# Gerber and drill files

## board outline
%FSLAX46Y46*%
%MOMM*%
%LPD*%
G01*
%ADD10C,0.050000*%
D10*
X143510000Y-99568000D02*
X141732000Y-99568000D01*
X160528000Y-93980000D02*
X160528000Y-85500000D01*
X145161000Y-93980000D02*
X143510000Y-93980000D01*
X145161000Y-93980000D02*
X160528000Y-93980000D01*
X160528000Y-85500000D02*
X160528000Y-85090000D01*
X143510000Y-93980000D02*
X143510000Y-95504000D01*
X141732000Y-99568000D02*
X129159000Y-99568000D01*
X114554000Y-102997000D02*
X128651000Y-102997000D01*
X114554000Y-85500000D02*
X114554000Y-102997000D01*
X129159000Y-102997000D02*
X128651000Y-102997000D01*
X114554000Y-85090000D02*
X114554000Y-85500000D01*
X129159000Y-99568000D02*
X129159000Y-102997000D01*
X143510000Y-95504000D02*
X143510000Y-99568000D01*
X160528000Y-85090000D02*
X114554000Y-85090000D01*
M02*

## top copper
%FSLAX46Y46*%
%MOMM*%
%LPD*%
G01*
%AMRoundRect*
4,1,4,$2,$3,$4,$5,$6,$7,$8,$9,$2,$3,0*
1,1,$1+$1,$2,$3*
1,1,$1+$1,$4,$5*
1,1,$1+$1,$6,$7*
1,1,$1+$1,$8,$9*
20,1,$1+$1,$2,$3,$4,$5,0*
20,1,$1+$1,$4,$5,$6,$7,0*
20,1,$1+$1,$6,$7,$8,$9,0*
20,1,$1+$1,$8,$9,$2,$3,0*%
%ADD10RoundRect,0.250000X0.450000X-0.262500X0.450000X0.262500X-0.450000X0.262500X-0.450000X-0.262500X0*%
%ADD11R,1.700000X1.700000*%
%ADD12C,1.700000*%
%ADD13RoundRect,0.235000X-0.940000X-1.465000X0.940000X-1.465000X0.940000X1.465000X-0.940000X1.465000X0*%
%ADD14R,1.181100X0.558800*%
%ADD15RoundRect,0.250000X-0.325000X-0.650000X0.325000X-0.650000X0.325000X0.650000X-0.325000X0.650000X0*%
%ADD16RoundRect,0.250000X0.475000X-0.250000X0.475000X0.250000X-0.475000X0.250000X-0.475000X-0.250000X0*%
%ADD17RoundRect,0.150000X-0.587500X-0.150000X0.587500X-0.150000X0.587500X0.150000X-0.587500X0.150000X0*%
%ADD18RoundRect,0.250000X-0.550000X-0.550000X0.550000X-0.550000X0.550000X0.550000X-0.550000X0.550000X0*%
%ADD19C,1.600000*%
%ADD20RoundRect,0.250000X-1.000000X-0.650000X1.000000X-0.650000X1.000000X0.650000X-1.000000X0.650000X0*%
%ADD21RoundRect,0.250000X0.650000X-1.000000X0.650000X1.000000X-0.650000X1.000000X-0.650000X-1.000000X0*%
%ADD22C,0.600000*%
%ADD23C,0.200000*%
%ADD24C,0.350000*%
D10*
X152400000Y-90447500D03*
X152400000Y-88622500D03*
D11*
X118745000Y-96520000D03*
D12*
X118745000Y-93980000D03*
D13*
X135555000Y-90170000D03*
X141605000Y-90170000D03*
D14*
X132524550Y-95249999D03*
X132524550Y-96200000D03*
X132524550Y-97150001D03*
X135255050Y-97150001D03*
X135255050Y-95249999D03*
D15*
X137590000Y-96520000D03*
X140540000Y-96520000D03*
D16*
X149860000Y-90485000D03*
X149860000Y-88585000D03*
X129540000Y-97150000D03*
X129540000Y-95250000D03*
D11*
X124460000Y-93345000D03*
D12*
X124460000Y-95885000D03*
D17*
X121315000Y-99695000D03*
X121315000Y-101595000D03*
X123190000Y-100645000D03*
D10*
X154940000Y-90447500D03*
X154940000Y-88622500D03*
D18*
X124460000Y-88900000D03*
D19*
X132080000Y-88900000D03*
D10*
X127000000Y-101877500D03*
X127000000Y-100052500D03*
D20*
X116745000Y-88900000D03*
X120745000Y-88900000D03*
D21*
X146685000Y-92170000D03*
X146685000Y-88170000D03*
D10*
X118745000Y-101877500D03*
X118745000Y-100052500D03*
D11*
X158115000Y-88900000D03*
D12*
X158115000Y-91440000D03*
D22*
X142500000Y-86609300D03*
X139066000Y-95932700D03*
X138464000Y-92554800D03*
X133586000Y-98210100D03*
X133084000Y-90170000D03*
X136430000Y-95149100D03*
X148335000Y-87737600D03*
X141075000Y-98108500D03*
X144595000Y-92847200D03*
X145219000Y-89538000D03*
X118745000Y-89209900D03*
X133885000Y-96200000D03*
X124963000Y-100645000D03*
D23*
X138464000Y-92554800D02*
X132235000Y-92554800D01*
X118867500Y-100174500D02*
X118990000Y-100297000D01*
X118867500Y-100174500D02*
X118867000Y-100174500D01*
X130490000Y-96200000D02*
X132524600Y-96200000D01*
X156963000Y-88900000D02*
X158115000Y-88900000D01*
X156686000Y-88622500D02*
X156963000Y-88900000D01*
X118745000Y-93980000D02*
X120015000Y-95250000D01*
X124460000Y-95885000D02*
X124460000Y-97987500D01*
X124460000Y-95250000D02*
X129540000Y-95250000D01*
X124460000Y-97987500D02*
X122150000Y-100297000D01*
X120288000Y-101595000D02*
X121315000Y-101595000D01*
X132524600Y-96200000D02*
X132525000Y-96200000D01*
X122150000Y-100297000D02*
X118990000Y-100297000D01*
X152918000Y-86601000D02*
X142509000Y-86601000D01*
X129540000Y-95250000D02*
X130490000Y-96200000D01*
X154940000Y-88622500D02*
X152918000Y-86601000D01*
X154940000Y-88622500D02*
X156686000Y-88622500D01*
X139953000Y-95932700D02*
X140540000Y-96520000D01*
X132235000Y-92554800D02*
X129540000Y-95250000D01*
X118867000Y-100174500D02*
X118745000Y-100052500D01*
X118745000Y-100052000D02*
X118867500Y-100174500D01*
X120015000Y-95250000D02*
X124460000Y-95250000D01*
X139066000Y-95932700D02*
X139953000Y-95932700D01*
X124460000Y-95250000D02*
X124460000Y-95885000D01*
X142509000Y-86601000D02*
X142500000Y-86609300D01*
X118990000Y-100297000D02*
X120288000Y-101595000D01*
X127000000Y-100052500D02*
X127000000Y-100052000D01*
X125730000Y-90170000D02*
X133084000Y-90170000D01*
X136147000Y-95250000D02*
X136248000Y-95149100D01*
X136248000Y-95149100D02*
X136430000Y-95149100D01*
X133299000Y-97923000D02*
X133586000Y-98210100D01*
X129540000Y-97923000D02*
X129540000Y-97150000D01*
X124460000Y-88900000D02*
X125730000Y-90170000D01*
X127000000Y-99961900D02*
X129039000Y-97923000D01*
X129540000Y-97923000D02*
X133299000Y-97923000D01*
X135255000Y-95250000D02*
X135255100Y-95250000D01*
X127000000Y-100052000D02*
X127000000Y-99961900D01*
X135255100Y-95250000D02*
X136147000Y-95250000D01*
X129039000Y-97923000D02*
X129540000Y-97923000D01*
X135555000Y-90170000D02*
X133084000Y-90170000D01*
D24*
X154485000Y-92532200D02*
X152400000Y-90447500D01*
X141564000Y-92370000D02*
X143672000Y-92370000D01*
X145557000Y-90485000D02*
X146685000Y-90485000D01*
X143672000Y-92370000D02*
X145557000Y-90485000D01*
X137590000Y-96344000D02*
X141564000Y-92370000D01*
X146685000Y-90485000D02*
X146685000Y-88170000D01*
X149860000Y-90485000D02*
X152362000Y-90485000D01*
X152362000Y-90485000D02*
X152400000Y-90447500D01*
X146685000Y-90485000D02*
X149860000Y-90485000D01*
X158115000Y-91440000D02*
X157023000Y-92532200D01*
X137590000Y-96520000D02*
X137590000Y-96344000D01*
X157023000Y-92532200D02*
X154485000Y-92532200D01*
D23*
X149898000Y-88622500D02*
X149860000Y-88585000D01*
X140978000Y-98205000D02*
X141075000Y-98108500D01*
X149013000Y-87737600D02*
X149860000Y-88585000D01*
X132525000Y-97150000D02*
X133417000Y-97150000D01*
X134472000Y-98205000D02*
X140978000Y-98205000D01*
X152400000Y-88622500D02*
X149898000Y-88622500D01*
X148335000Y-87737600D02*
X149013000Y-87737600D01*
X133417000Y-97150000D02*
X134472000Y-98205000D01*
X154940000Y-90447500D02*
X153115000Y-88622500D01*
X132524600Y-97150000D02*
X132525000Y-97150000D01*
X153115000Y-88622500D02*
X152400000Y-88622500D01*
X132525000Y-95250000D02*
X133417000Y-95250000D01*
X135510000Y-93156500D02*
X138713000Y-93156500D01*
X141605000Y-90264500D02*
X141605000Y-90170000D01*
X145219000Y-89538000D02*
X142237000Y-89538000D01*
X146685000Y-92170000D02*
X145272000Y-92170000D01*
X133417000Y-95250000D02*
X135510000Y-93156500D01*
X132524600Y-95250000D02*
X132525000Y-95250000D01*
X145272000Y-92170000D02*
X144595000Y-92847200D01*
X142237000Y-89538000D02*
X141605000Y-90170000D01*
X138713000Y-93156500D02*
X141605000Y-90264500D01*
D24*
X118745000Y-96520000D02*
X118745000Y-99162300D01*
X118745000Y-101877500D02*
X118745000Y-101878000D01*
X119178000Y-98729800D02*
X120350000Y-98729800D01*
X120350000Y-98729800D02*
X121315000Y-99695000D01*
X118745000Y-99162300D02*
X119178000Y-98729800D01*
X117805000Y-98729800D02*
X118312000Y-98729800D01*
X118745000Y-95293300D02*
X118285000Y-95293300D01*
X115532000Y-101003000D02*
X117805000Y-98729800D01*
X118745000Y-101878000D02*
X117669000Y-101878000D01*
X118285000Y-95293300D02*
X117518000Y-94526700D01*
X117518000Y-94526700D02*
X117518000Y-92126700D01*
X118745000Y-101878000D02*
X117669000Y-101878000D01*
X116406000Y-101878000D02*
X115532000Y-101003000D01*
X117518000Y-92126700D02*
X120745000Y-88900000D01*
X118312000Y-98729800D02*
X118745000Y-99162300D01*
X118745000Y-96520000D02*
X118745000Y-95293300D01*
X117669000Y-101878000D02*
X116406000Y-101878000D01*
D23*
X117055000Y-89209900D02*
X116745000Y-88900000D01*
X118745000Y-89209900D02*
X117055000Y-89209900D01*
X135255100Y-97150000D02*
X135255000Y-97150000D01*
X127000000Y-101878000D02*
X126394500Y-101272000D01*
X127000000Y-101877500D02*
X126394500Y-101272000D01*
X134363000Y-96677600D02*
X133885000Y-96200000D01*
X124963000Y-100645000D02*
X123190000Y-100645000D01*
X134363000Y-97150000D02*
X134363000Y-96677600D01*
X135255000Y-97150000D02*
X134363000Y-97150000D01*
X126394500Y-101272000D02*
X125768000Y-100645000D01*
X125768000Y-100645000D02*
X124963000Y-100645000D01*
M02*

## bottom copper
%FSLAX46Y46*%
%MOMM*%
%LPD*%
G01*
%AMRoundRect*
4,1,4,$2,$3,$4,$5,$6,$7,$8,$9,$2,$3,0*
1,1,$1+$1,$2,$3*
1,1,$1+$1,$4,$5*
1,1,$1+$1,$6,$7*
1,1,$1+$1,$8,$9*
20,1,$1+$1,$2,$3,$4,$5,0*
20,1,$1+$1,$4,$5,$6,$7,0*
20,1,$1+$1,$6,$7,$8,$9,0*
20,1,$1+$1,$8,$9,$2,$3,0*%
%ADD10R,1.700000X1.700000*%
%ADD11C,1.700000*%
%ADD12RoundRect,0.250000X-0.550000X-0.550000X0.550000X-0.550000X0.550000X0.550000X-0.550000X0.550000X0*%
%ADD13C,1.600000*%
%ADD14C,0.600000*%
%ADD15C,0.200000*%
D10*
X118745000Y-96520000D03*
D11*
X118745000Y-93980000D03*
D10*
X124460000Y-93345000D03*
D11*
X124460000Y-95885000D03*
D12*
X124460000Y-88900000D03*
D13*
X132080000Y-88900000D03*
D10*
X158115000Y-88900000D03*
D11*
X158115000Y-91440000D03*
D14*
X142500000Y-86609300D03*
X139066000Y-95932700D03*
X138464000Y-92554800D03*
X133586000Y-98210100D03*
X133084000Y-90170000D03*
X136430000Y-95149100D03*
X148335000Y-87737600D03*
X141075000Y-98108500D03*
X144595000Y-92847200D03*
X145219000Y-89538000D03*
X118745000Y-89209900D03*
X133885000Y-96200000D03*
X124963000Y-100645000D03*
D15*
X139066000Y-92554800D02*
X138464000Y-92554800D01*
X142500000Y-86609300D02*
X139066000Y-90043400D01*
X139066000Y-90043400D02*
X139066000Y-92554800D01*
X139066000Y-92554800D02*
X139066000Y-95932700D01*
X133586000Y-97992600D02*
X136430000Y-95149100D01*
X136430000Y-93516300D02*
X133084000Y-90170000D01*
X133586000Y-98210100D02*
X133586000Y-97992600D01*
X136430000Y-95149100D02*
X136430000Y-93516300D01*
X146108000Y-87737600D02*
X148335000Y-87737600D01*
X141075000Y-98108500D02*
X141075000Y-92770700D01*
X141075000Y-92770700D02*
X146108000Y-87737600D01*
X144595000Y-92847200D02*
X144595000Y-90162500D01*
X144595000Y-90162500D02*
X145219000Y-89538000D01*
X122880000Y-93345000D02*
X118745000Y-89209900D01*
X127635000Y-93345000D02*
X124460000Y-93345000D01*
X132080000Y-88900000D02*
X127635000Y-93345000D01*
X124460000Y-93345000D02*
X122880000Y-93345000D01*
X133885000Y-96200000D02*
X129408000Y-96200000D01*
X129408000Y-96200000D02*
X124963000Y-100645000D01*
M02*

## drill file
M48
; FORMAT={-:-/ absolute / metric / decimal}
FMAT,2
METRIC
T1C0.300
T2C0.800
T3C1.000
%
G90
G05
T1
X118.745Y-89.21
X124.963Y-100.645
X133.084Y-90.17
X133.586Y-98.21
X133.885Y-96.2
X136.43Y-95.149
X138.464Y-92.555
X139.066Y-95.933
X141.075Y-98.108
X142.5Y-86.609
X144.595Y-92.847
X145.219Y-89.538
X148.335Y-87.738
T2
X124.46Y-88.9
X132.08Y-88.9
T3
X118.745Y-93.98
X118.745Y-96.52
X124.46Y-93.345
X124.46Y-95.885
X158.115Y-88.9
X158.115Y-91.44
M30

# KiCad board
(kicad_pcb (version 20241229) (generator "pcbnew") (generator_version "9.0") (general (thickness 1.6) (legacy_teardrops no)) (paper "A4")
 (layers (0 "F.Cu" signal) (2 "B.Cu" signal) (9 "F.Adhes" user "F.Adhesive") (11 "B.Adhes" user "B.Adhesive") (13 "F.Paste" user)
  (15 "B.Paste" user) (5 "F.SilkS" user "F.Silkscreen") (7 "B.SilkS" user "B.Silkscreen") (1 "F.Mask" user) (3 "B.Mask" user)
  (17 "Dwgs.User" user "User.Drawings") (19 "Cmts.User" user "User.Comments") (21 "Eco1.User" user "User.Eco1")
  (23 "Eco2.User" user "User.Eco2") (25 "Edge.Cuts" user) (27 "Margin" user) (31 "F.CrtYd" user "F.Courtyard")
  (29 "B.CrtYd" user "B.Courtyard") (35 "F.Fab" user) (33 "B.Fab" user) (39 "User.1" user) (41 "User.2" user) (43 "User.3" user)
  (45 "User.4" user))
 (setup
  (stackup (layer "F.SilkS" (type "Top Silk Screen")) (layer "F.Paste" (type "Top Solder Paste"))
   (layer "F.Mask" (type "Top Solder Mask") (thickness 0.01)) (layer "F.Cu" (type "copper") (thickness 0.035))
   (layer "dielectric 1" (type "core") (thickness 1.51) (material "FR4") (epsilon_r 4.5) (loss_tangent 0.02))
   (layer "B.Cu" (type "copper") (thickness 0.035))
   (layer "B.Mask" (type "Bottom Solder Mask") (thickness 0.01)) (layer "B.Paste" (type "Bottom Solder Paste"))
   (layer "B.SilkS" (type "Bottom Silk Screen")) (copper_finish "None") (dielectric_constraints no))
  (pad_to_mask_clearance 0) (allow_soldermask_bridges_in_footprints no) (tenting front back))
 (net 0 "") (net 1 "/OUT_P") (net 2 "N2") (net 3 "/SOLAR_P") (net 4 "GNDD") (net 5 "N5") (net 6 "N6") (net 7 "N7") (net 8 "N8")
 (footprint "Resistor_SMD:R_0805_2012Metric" (layer "F.Cu") (at 152.4 89.535 90)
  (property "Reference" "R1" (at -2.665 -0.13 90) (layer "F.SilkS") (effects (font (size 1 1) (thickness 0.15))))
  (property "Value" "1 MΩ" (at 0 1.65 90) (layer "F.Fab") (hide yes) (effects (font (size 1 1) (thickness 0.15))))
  (pad "1" smd roundrect (at -0.9125 0 90) (size 1.025 1.4) (layers "F.Cu" "F.Mask" "F.Paste") (roundrect_rratio 0.243902) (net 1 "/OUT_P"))
  (pad "2" smd roundrect (at 0.9125 0 90) (size 1.025 1.4) (layers "F.Cu" "F.Mask" "F.Paste") (roundrect_rratio 0.243902) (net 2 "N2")))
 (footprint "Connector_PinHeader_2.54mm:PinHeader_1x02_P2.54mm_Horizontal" (layer "F.Cu") (at 118.745 96.52 180)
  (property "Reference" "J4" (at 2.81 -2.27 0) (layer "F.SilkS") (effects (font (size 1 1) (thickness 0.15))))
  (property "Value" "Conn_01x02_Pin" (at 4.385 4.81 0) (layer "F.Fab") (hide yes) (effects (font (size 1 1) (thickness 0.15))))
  (pad "1" thru_hole rect (at 0 0 180) (size 1.7 1.7) (drill 1) (layers "*.Cu" "*.Mask") (remove_unused_layers no) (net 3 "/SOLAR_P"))
  (pad "2" thru_hole circle (at 0 2.54 180) (size 1.7 1.7) (drill 1) (layers "*.Cu" "*.Mask") (remove_unused_layers no) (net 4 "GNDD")))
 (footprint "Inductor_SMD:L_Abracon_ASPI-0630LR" (layer "F.Cu") (at 138.58 90.17)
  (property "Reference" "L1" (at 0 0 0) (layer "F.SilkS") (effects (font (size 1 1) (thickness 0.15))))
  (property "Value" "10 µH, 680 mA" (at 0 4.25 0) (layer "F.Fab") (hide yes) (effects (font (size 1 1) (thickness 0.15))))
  (pad "1" smd roundrect (at -3.025 0) (size 2.35 3.4) (layers "F.Cu" "F.Mask" "F.Paste") (roundrect_rratio 0.1) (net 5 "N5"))
  (pad "2" smd roundrect (at 3.025 0) (size 2.35 3.4) (layers "F.Cu" "F.Mask" "F.Paste") (roundrect_rratio 0.1) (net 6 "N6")))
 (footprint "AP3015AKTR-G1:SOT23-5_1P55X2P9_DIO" (layer "F.Cu") (at 133.8898 96.2)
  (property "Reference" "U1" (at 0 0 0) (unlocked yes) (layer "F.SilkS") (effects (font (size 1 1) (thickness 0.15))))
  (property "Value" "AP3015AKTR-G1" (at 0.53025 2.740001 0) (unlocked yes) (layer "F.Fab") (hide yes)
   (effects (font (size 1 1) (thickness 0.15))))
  (pad "1" smd rect (at -1.36525 -0.950001) (size 1.1811 0.5588) (layers "F.Cu" "F.Mask" "F.Paste") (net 6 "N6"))
  (pad "2" smd rect (at -1.36525 0) (size 1.1811 0.5588) (layers "F.Cu" "F.Mask" "F.Paste") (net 4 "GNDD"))
  (pad "3" smd rect (at -1.36525 0.950001) (size 1.1811 0.5588) (layers "F.Cu" "F.Mask" "F.Paste") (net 2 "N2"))
  (pad "4" smd rect (at 1.36525 0.950001) (size 1.1811 0.5588) (layers "F.Cu" "F.Mask" "F.Paste") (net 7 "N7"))
  (pad "5" smd rect (at 1.36525 -0.950001) (size 1.1811 0.5588) (layers "F.Cu" "F.Mask" "F.Paste") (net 5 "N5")))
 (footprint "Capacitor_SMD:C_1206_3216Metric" (layer "F.Cu") (at 139.065 96.52)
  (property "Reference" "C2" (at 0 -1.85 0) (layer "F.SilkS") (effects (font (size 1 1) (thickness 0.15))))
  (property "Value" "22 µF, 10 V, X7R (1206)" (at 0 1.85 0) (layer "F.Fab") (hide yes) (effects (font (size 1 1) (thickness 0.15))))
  (pad "1" smd roundrect (at -1.475 0) (size 1.15 1.8) (layers "F.Cu" "F.Mask" "F.Paste") (roundrect_rratio 0.217391) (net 1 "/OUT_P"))
  (pad "2" smd roundrect (at 1.475 0) (size 1.15 1.8) (layers "F.Cu" "F.Mask" "F.Paste") (roundrect_rratio 0.217391) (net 4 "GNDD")))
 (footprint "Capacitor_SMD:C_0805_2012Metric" (layer "F.Cu") (at 149.86 89.535 90)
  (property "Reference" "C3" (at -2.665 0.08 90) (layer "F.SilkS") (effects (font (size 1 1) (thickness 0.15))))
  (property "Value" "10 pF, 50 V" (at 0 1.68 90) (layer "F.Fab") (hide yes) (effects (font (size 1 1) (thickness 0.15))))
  (pad "1" smd roundrect (at -0.95 0 90) (size 1 1.45) (layers "F.Cu" "F.Mask" "F.Paste") (roundrect_rratio 0.25) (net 1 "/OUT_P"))
  (pad "2" smd roundrect (at 0.95 0 90) (size 1 1.45) (layers "F.Cu" "F.Mask" "F.Paste") (roundrect_rratio 0.25) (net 2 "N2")))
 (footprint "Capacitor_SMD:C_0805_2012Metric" (layer "F.Cu") (at 129.54 96.2 90)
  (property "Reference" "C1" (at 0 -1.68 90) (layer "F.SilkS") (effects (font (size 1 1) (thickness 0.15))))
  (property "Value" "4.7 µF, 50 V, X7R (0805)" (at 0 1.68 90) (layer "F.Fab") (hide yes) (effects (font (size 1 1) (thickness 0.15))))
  (pad "1" smd roundrect (at -0.95 0 90) (size 1 1.45) (layers "F.Cu" "F.Mask" "F.Paste") (roundrect_rratio 0.25) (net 5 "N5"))
  (pad "2" smd roundrect (at 0.95 0 90) (size 1 1.45) (layers "F.Cu" "F.Mask" "F.Paste") (roundrect_rratio 0.25) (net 4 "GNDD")))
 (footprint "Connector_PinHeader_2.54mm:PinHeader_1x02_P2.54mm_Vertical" (layer "F.Cu") (at 124.46 93.345)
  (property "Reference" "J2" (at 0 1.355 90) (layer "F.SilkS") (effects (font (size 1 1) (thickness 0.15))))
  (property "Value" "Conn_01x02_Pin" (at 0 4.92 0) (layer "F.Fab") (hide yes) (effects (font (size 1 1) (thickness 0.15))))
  (pad "1" thru_hole rect (at 0 0) (size 1.7 1.7) (drill 1) (layers "*.Cu" "*.Mask") (remove_unused_layers no) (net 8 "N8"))
  (pad "2" thru_hole circle (at 0 2.54) (size 1.7 1.7) (drill 1) (layers "*.Cu" "*.Mask") (remove_unused_layers no) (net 4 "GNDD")))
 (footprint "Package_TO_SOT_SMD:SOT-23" (layer "F.Cu") (at 122.2525 100.645)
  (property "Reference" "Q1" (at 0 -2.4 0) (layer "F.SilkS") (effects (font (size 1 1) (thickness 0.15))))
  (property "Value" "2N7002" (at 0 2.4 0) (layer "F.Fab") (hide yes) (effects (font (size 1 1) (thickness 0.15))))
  (pad "1" smd roundrect (at -0.9375 -0.95) (size 1.475 0.6) (layers "F.Cu" "F.Mask" "F.Paste") (roundrect_rratio 0.25) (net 3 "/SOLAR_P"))
  (pad "2" smd roundrect (at -0.9375 0.95) (size 1.475 0.6) (layers "F.Cu" "F.Mask" "F.Paste") (roundrect_rratio 0.25) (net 4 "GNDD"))
  (pad "3" smd roundrect (at 0.9375 0) (size 1.475 0.6) (layers "F.Cu" "F.Mask" "F.Paste") (roundrect_rratio 0.25) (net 7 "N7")))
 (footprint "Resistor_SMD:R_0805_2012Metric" (layer "F.Cu") (at 154.94 89.535 90)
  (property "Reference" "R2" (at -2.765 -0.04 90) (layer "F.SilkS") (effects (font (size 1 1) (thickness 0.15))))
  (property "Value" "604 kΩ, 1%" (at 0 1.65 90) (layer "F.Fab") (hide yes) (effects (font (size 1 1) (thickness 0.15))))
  (pad "1" smd roundrect (at -0.9125 0 90) (size 1.025 1.4) (layers "F.Cu" "F.Mask" "F.Paste") (roundrect_rratio 0.243902) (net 2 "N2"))
  (pad "2" smd roundrect (at 0.9125 0 90) (size 1.025 1.4) (layers "F.Cu" "F.Mask" "F.Paste") (roundrect_rratio 0.243902) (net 4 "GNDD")))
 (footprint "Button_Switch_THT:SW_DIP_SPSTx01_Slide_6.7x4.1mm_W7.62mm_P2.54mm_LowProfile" (layer "F.Cu") (at 124.46 88.9)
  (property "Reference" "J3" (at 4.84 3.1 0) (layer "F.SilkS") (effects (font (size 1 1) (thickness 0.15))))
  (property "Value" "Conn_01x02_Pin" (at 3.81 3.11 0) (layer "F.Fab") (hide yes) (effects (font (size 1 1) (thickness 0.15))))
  (pad "1" thru_hole roundrect (at 0 0) (size 1.6 1.6) (drill 0.8) (layers "*.Cu" "*.Mask") (remove_unused_layers no)
   (roundrect_rratio 0.15625) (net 5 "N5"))
  (pad "2" thru_hole circle (at 7.62 0) (size 1.6 1.6) (drill 0.8) (layers "*.Cu" "*.Mask") (remove_unused_layers no) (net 8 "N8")))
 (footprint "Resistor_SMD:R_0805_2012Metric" (layer "F.Cu") (at 127 100.965 90)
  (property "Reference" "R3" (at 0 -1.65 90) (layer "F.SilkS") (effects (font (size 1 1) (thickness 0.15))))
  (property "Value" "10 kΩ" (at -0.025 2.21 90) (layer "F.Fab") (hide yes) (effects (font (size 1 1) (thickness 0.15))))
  (pad "1" smd roundrect (at -0.9125 0 90) (size 1.025 1.4) (layers "F.Cu" "F.Mask" "F.Paste") (roundrect_rratio 0.243902) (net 7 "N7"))
  (pad "2" smd roundrect (at 0.9125 0 90) (size 1.025 1.4) (layers "F.Cu" "F.Mask" "F.Paste") (roundrect_rratio 0.243902) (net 5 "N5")))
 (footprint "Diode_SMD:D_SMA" (layer "F.Cu") (at 118.745 88.9)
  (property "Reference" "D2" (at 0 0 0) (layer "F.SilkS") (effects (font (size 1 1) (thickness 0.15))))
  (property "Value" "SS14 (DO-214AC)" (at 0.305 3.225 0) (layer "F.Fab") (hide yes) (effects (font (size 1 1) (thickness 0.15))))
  (pad "1" smd roundrect (at -2 0) (size 2.5 1.8) (layers "F.Cu" "F.Mask" "F.Paste") (roundrect_rratio 0.1388888889) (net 8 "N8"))
  (pad "2" smd roundrect (at 2 0) (size 2.5 1.8) (layers "F.Cu" "F.Mask" "F.Paste") (roundrect_rratio 0.1388888889) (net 3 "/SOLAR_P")))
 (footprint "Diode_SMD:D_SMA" (layer "F.Cu") (at 146.685 90.17 90)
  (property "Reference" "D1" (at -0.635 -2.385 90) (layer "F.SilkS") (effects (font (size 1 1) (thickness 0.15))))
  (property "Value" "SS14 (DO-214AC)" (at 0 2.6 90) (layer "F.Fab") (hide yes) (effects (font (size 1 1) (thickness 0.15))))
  (pad "1" smd roundrect (at -2 0 90) (size 2.5 1.8) (layers "F.Cu" "F.Mask" "F.Paste") (roundrect_rratio 0.1388888889) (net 6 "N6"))
  (pad "2" smd roundrect (at 2 0 90) (size 2.5 1.8) (layers "F.Cu" "F.Mask" "F.Paste") (roundrect_rratio 0.1388888889) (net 1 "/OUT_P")))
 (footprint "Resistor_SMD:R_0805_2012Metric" (layer "F.Cu") (at 118.745 100.965 90)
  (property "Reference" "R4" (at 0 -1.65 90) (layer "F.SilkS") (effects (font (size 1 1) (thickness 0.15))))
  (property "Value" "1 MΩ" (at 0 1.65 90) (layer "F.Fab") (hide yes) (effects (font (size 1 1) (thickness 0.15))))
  (pad "1" smd roundrect (at -0.9125 0 90) (size 1.025 1.4) (layers "F.Cu" "F.Mask" "F.Paste") (roundrect_rratio 0.243902)
   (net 3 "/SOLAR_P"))
  (pad "2" smd roundrect (at 0.9125 0 90) (size 1.025 1.4) (layers "F.Cu" "F.Mask" "F.Paste") (roundrect_rratio 0.243902) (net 4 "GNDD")))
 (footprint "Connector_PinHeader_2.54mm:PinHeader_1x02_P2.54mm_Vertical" (layer "F.Cu") (at 158.115 88.9)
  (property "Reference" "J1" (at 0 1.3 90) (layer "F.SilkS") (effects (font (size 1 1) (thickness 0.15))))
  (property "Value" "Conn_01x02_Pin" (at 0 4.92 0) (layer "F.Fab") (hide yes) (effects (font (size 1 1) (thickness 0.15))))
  (pad "1" thru_hole rect (at 0 0) (size 1.7 1.7) (drill 1) (layers "*.Cu" "*.Mask") (remove_unused_layers no) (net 4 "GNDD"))
  (pad "2" thru_hole circle (at 0 2.54) (size 1.7 1.7) (drill 1) (layers "*.Cu" "*.Mask") (remove_unused_layers no) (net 1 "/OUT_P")))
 (gr_line (start 143.51 99.568) (end 141.732 99.568) (stroke (width 0.05) (type default)) (layer "Edge.Cuts"))
 (gr_line (start 160.528 93.98) (end 160.528 85.5) (stroke (width 0.05) (type default)) (layer "Edge.Cuts"))
 (gr_line (start 145.161 93.98) (end 143.51 93.98) (stroke (width 0.05) (type default)) (layer "Edge.Cuts"))
 (gr_line (start 145.161 93.98) (end 160.528 93.98) (stroke (width 0.05) (type default)) (layer "Edge.Cuts"))
 (gr_line (start 160.528 85.5) (end 160.528 85.09) (stroke (width 0.05) (type default)) (layer "Edge.Cuts"))
 (gr_line (start 143.51 93.98) (end 143.51 95.504) (stroke (width 0.05) (type default)) (layer "Edge.Cuts"))
 (gr_line (start 141.732 99.568) (end 129.159 99.568) (stroke (width 0.05) (type default)) (layer "Edge.Cuts"))
 (gr_line (start 114.554 102.997) (end 128.651 102.997) (stroke (width 0.05) (type default)) (layer "Edge.Cuts"))
 (gr_line (start 114.554 85.5) (end 114.554 102.997) (stroke (width 0.05) (type default)) (layer "Edge.Cuts"))
 (gr_line (start 129.159 102.997) (end 128.651 102.997) (stroke (width 0.05) (type default)) (layer "Edge.Cuts"))
 (gr_line (start 114.554 85.09) (end 114.554 85.5) (stroke (width 0.05) (type default)) (layer "Edge.Cuts"))
 (gr_line (start 129.159 99.568) (end 129.159 102.997) (stroke (width 0.05) (type default)) (layer "Edge.Cuts"))
 (gr_line (start 143.51 95.504) (end 143.51 99.568) (stroke (width 0.05) (type default)) (layer "Edge.Cuts"))
 (gr_line (start 160.528 85.09) (end 114.554 85.09) (stroke (width 0.05) (type default)) (layer "Edge.Cuts"))
 (segment (start 138.464 92.5548) (end 132.235 92.5548) (width 0.2) (layer "F.Cu") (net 4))
 (segment (start 118.8675 100.1745) (end 118.99 100.297) (width 0.2) (layer "F.Cu") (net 4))
 (segment (start 118.8675 100.1745) (end 118.867 100.1745) (width 0.2) (layer "F.Cu") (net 4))
 (segment (start 130.49 96.2) (end 132.5246 96.2) (width 0.2) (layer "F.Cu") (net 4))
 (segment (start 156.963 88.9) (end 158.115 88.9) (width 0.2) (layer "F.Cu") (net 4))
 (segment (start 156.686 88.6225) (end 156.963 88.9) (width 0.2) (layer "F.Cu") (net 4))
 (segment (start 118.745 93.98) (end 120.015 95.25) (width 0.2) (layer "F.Cu") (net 4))
 (segment (start 124.46 95.885) (end 124.46 97.9875) (width 0.2) (layer "F.Cu") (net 4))
 (segment (start 124.46 95.25) (end 129.54 95.25) (width 0.2) (layer "F.Cu") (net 4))
 (segment (start 124.46 97.9875) (end 122.15 100.297) (width 0.2) (layer "F.Cu") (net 4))
 (segment (start 120.288 101.595) (end 121.315 101.595) (width 0.2) (layer "F.Cu") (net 4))
 (segment (start 132.5246 96.2) (end 132.525 96.2) (width 0.2) (layer "F.Cu") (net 4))
 (segment (start 122.15 100.297) (end 118.99 100.297) (width 0.2) (layer "F.Cu") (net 4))
 (segment (start 152.918 86.601) (end 142.509 86.601) (width 0.2) (layer "F.Cu") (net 4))
 (segment (start 129.54 95.25) (end 130.49 96.2) (width 0.2) (layer "F.Cu") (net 4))
 (segment (start 154.94 88.6225) (end 152.918 86.601) (width 0.2) (layer "F.Cu") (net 4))
 (segment (start 154.94 88.6225) (end 156.686 88.6225) (width 0.2) (layer "F.Cu") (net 4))
 (segment (start 139.953 95.9327) (end 140.54 96.52) (width 0.2) (layer "F.Cu") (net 4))
 (segment (start 132.235 92.5548) (end 129.54 95.25) (width 0.2) (layer "F.Cu") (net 4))
 (segment (start 118.867 100.1745) (end 118.745 100.0525) (width 0.2) (layer "F.Cu") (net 4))
 (segment (start 118.745 100.052) (end 118.8675 100.1745) (width 0.2) (layer "F.Cu") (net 4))
 (segment (start 120.015 95.25) (end 124.46 95.25) (width 0.2) (layer "F.Cu") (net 4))
 (segment (start 139.066 95.9327) (end 139.953 95.9327) (width 0.2) (layer "F.Cu") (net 4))
 (segment (start 124.46 95.25) (end 124.46 95.885) (width 0.2) (layer "F.Cu") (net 4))
 (segment (start 142.509 86.601) (end 142.5 86.6093) (width 0.2) (layer "F.Cu") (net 4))
 (segment (start 118.99 100.297) (end 120.288 101.595) (width 0.2) (layer "F.Cu") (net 4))
 (via (at 142.5 86.6093) (size 0.6) (drill 0.3) (layers "F.Cu" "B.Cu") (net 4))
 (via (at 139.066 95.9327) (size 0.6) (drill 0.3) (layers "F.Cu" "B.Cu") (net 4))
 (via (at 138.464 92.5548) (size 0.6) (drill 0.3) (layers "F.Cu" "B.Cu") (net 4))
 (segment (start 139.066 92.5548) (end 138.464 92.5548) (width 0.2) (layer "B.Cu") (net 4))
 (segment (start 142.5 86.6093) (end 139.066 90.0434) (width 0.2) (layer "B.Cu") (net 4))
 (segment (start 139.066 90.0434) (end 139.066 92.5548) (width 0.2) (layer "B.Cu") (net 4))
 (segment (start 139.066 92.5548) (end 139.066 95.9327) (width 0.2) (layer "B.Cu") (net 4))
 (segment (start 127 100.0525) (end 127 100.052) (width 0.2) (layer "F.Cu") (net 5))
 (segment (start 125.73 90.17) (end 133.084 90.17) (width 0.2) (layer "F.Cu") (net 5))
 (segment (start 136.147 95.25) (end 136.248 95.1491) (width 0.2) (layer "F.Cu") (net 5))
 (segment (start 136.248 95.1491) (end 136.43 95.1491) (width 0.2) (layer "F.Cu") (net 5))
 (segment (start 133.299 97.923) (end 133.586 98.2101) (width 0.2) (layer "F.Cu") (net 5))
 (segment (start 129.54 97.923) (end 129.54 97.15) (width 0.2) (layer "F.Cu") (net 5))
 (segment (start 124.46 88.9) (end 125.73 90.17) (width 0.2) (layer "F.Cu") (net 5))
 (segment (start 127 99.9619) (end 129.039 97.923) (width 0.2) (layer "F.Cu") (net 5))
 (segment (start 129.54 97.923) (end 133.299 97.923) (width 0.2) (layer "F.Cu") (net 5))
 (segment (start 135.255 95.25) (end 135.2551 95.25) (width 0.2) (layer "F.Cu") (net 5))
 (segment (start 127 100.052) (end 127 99.9619) (width 0.2) (layer "F.Cu") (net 5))
 (segment (start 135.2551 95.25) (end 136.147 95.25) (width 0.2) (layer "F.Cu") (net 5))
 (segment (start 129.039 97.923) (end 129.54 97.923) (width 0.2) (layer "F.Cu") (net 5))
 (segment (start 135.555 90.17) (end 133.084 90.17) (width 0.2) (layer "F.Cu") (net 5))
 (via (at 133.586 98.2101) (size 0.6) (drill 0.3) (layers "F.Cu" "B.Cu") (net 5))
 (via (at 133.084 90.17) (size 0.6) (drill 0.3) (layers "F.Cu" "B.Cu") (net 5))
 (via (at 136.43 95.1491) (size 0.6) (drill 0.3) (layers "F.Cu" "B.Cu") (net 5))
 (segment (start 133.586 97.9926) (end 136.43 95.1491) (width 0.2) (layer "B.Cu") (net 5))
 (segment (start 136.43 93.5163) (end 133.084 90.17) (width 0.2) (layer "B.Cu") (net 5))
 (segment (start 133.586 98.2101) (end 133.586 97.9926) (width 0.2) (layer "B.Cu") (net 5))
 (segment (start 136.43 95.1491) (end 136.43 93.5163) (width 0.2) (layer "B.Cu") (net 5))
 (segment (start 154.485 92.5322) (end 152.4 90.4475) (width 0.35) (layer "F.Cu") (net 1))
 (segment (start 141.564 92.37) (end 143.672 92.37) (width 0.35) (layer "F.Cu") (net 1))
 (segment (start 145.557 90.485) (end 146.685 90.485) (width 0.35) (layer "F.Cu") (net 1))
 (segment (start 143.672 92.37) (end 145.557 90.485) (width 0.35) (layer "F.Cu") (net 1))
 (segment (start 137.59 96.344) (end 141.564 92.37) (width 0.35) (layer "F.Cu") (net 1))
 (segment (start 146.685 90.485) (end 146.685 88.17) (width 0.35) (layer "F.Cu") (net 1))
 (segment (start 149.86 90.485) (end 152.362 90.485) (width 0.35) (layer "F.Cu") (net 1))
 (segment (start 152.362 90.485) (end 152.4 90.4475) (width 0.35) (layer "F.Cu") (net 1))
 (segment (start 146.685 90.485) (end 149.86 90.485) (width 0.35) (layer "F.Cu") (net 1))
 (segment (start 158.115 91.44) (end 157.023 92.5322) (width 0.35) (layer "F.Cu") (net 1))
 (segment (start 137.59 96.52) (end 137.59 96.344) (width 0.35) (layer "F.Cu") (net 1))
 (segment (start 157.023 92.5322) (end 154.485 92.5322) (width 0.35) (layer "F.Cu") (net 1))
 (segment (start 149.898 88.6225) (end 149.86 88.585) (width 0.2) (layer "F.Cu") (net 2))
 (segment (start 140.978 98.205) (end 141.075 98.1085) (width 0.2) (layer "F.Cu") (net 2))
 (segment (start 149.013 87.7376) (end 149.86 88.585) (width 0.2) (layer "F.Cu") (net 2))
 (segment (start 132.525 97.15) (end 133.417 97.15) (width 0.2) (layer "F.Cu") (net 2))
 (segment (start 134.472 98.205) (end 140.978 98.205) (width 0.2) (layer "F.Cu") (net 2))
 (segment (start 152.4 88.6225) (end 149.898 88.6225) (width 0.2) (layer "F.Cu") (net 2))
 (segment (start 148.335 87.7376) (end 149.013 87.7376) (width 0.2) (layer "F.Cu") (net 2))
 (segment (start 133.417 97.15) (end 134.472 98.205) (width 0.2) (layer "F.Cu") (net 2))
 (segment (start 154.94 90.4475) (end 153.115 88.6225) (width 0.2) (layer "F.Cu") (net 2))
 (segment (start 132.5246 97.15) (end 132.525 97.15) (width 0.2) (layer "F.Cu") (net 2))
 (segment (start 153.115 88.6225) (end 152.4 88.6225) (width 0.2) (layer "F.Cu") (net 2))
 (via (at 148.335 87.7376) (size 0.6) (drill 0.3) (layers "F.Cu" "B.Cu") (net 2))
 (via (at 141.075 98.1085) (size 0.6) (drill 0.3) (layers "F.Cu" "B.Cu") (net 2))
 (segment (start 146.108 87.7376) (end 148.335 87.7376) (width 0.2) (layer "B.Cu") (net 2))
 (segment (start 141.075 98.1085) (end 141.075 92.7707) (width 0.2) (layer "B.Cu") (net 2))
 (segment (start 141.075 92.7707) (end 146.108 87.7376) (width 0.2) (layer "B.Cu") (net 2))
 (segment (start 132.525 95.25) (end 133.417 95.25) (width 0.2) (layer "F.Cu") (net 6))
 (segment (start 135.51 93.1565) (end 138.713 93.1565) (width 0.2) (layer "F.Cu") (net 6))
 (segment (start 141.605 90.2645) (end 141.605 90.17) (width 0.2) (layer "F.Cu") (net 6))
 (segment (start 145.219 89.538) (end 142.237 89.538) (width 0.2) (layer "F.Cu") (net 6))
 (segment (start 146.685 92.17) (end 145.272 92.17) (width 0.2) (layer "F.Cu") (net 6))
 (segment (start 133.417 95.25) (end 135.51 93.1565) (width 0.2) (layer "F.Cu") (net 6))
 (segment (start 132.5246 95.25) (end 132.525 95.25) (width 0.2) (layer "F.Cu") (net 6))
 (segment (start 145.272 92.17) (end 144.595 92.8472) (width 0.2) (layer "F.Cu") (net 6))
 (segment (start 142.237 89.538) (end 141.605 90.17) (width 0.2) (layer "F.Cu") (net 6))
 (segment (start 138.713 93.1565) (end 141.605 90.2645) (width 0.2) (layer "F.Cu") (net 6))
 (via (at 144.595 92.8472) (size 0.6) (drill 0.3) (layers "F.Cu" "B.Cu") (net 6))
 (via (at 145.219 89.538) (size 0.6) (drill 0.3) (layers "F.Cu" "B.Cu") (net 6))
 (segment (start 144.595 92.8472) (end 144.595 90.1625) (width 0.2) (layer "B.Cu") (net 6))
 (segment (start 144.595 90.1625) (end 145.219 89.538) (width 0.2) (layer "B.Cu") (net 6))
 (segment (start 118.745 96.52) (end 118.745 99.1623) (width 0.35) (layer "F.Cu") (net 3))
 (segment (start 118.745 101.8775) (end 118.745 101.878) (width 0.35) (layer "F.Cu") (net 3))
 (segment (start 119.178 98.7298) (end 120.35 98.7298) (width 0.35) (layer "F.Cu") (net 3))
 (segment (start 120.35 98.7298) (end 121.315 99.695) (width 0.35) (layer "F.Cu") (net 3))
 (segment (start 118.745 99.1623) (end 119.178 98.7298) (width 0.35) (layer "F.Cu") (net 3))
 (segment (start 117.805 98.7298) (end 118.312 98.7298) (width 0.35) (layer "F.Cu") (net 3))
 (segment (start 118.745 95.2933) (end 118.285 95.2933) (width 0.35) (layer "F.Cu") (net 3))
 (segment (start 115.532 101.003) (end 117.805 98.7298) (width 0.35) (layer "F.Cu") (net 3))
 (segment (start 118.745 101.878) (end 117.669 101.878) (width 0.35) (layer "F.Cu") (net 3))
 (segment (start 118.285 95.2933) (end 117.518 94.5267) (width 0.35) (layer "F.Cu") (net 3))
 (segment (start 117.518 94.5267) (end 117.518 92.1267) (width 0.35) (layer "F.Cu") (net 3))
 (segment (start 118.745 101.878) (end 117.669 101.878) (width 0.35) (layer "F.Cu") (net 3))
 (segment (start 116.406 101.878) (end 115.532 101.003) (width 0.35) (layer "F.Cu") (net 3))
 (segment (start 117.518 92.1267) (end 120.745 88.9) (width 0.35) (layer "F.Cu") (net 3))
 (segment (start 118.312 98.7298) (end 118.745 99.1623) (width 0.35) (layer "F.Cu") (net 3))
 (segment (start 118.745 96.52) (end 118.745 95.2933) (width 0.35) (layer "F.Cu") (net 3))
 (segment (start 117.669 101.878) (end 116.406 101.878) (width 0.35) (layer "F.Cu") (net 3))
 (segment (start 117.055 89.2099) (end 116.745 88.9) (width 0.2) (layer "F.Cu") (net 8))
 (segment (start 118.745 89.2099) (end 117.055 89.2099) (width 0.2) (layer "F.Cu") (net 8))
 (via (at 118.745 89.2099) (size 0.6) (drill 0.3) (layers "F.Cu" "B.Cu") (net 8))
 (segment (start 122.88 93.345) (end 118.745 89.2099) (width 0.2) (layer "B.Cu") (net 8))
 (segment (start 127.635 93.345) (end 124.46 93.345) (width 0.2) (layer "B.Cu") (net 8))
 (segment (start 132.08 88.9) (end 127.635 93.345) (width 0.2) (layer "B.Cu") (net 8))
 (segment (start 124.46 93.345) (end 122.88 93.345) (width 0.2) (layer "B.Cu") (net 8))
 (segment (start 135.2551 97.15) (end 135.255 97.15) (width 0.2) (layer "F.Cu") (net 7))
 (segment (start 127 101.878) (end 126.3945 101.272) (width 0.2) (layer "F.Cu") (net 7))
 (segment (start 127 101.8775) (end 126.3945 101.272) (width 0.2) (layer "F.Cu") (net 7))
 (segment (start 134.363 96.6776) (end 133.885 96.2) (width 0.2) (layer "F.Cu") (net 7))
 (segment (start 124.963 100.645) (end 123.19 100.645) (width 0.2) (layer "F.Cu") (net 7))
 (segment (start 134.363 97.15) (end 134.363 96.6776) (width 0.2) (layer "F.Cu") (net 7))
 (segment (start 135.255 97.15) (end 134.363 97.15) (width 0.2) (layer "F.Cu") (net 7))
 (segment (start 126.3945 101.272) (end 125.768 100.645) (width 0.2) (layer "F.Cu") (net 7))
 (segment (start 125.768 100.645) (end 124.963 100.645) (width 0.2) (layer "F.Cu") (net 7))
 (via (at 133.885 96.2) (size 0.6) (drill 0.3) (layers "F.Cu" "B.Cu") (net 7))
 (via (at 124.963 100.645) (size 0.6) (drill 0.3) (layers "F.Cu" "B.Cu") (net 7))
 (segment (start 133.885 96.2) (end 129.408 96.2) (width 0.2) (layer "B.Cu") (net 7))
 (segment (start 129.408 96.2) (end 124.963 100.645) (width 0.2) (layer "B.Cu") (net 7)))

